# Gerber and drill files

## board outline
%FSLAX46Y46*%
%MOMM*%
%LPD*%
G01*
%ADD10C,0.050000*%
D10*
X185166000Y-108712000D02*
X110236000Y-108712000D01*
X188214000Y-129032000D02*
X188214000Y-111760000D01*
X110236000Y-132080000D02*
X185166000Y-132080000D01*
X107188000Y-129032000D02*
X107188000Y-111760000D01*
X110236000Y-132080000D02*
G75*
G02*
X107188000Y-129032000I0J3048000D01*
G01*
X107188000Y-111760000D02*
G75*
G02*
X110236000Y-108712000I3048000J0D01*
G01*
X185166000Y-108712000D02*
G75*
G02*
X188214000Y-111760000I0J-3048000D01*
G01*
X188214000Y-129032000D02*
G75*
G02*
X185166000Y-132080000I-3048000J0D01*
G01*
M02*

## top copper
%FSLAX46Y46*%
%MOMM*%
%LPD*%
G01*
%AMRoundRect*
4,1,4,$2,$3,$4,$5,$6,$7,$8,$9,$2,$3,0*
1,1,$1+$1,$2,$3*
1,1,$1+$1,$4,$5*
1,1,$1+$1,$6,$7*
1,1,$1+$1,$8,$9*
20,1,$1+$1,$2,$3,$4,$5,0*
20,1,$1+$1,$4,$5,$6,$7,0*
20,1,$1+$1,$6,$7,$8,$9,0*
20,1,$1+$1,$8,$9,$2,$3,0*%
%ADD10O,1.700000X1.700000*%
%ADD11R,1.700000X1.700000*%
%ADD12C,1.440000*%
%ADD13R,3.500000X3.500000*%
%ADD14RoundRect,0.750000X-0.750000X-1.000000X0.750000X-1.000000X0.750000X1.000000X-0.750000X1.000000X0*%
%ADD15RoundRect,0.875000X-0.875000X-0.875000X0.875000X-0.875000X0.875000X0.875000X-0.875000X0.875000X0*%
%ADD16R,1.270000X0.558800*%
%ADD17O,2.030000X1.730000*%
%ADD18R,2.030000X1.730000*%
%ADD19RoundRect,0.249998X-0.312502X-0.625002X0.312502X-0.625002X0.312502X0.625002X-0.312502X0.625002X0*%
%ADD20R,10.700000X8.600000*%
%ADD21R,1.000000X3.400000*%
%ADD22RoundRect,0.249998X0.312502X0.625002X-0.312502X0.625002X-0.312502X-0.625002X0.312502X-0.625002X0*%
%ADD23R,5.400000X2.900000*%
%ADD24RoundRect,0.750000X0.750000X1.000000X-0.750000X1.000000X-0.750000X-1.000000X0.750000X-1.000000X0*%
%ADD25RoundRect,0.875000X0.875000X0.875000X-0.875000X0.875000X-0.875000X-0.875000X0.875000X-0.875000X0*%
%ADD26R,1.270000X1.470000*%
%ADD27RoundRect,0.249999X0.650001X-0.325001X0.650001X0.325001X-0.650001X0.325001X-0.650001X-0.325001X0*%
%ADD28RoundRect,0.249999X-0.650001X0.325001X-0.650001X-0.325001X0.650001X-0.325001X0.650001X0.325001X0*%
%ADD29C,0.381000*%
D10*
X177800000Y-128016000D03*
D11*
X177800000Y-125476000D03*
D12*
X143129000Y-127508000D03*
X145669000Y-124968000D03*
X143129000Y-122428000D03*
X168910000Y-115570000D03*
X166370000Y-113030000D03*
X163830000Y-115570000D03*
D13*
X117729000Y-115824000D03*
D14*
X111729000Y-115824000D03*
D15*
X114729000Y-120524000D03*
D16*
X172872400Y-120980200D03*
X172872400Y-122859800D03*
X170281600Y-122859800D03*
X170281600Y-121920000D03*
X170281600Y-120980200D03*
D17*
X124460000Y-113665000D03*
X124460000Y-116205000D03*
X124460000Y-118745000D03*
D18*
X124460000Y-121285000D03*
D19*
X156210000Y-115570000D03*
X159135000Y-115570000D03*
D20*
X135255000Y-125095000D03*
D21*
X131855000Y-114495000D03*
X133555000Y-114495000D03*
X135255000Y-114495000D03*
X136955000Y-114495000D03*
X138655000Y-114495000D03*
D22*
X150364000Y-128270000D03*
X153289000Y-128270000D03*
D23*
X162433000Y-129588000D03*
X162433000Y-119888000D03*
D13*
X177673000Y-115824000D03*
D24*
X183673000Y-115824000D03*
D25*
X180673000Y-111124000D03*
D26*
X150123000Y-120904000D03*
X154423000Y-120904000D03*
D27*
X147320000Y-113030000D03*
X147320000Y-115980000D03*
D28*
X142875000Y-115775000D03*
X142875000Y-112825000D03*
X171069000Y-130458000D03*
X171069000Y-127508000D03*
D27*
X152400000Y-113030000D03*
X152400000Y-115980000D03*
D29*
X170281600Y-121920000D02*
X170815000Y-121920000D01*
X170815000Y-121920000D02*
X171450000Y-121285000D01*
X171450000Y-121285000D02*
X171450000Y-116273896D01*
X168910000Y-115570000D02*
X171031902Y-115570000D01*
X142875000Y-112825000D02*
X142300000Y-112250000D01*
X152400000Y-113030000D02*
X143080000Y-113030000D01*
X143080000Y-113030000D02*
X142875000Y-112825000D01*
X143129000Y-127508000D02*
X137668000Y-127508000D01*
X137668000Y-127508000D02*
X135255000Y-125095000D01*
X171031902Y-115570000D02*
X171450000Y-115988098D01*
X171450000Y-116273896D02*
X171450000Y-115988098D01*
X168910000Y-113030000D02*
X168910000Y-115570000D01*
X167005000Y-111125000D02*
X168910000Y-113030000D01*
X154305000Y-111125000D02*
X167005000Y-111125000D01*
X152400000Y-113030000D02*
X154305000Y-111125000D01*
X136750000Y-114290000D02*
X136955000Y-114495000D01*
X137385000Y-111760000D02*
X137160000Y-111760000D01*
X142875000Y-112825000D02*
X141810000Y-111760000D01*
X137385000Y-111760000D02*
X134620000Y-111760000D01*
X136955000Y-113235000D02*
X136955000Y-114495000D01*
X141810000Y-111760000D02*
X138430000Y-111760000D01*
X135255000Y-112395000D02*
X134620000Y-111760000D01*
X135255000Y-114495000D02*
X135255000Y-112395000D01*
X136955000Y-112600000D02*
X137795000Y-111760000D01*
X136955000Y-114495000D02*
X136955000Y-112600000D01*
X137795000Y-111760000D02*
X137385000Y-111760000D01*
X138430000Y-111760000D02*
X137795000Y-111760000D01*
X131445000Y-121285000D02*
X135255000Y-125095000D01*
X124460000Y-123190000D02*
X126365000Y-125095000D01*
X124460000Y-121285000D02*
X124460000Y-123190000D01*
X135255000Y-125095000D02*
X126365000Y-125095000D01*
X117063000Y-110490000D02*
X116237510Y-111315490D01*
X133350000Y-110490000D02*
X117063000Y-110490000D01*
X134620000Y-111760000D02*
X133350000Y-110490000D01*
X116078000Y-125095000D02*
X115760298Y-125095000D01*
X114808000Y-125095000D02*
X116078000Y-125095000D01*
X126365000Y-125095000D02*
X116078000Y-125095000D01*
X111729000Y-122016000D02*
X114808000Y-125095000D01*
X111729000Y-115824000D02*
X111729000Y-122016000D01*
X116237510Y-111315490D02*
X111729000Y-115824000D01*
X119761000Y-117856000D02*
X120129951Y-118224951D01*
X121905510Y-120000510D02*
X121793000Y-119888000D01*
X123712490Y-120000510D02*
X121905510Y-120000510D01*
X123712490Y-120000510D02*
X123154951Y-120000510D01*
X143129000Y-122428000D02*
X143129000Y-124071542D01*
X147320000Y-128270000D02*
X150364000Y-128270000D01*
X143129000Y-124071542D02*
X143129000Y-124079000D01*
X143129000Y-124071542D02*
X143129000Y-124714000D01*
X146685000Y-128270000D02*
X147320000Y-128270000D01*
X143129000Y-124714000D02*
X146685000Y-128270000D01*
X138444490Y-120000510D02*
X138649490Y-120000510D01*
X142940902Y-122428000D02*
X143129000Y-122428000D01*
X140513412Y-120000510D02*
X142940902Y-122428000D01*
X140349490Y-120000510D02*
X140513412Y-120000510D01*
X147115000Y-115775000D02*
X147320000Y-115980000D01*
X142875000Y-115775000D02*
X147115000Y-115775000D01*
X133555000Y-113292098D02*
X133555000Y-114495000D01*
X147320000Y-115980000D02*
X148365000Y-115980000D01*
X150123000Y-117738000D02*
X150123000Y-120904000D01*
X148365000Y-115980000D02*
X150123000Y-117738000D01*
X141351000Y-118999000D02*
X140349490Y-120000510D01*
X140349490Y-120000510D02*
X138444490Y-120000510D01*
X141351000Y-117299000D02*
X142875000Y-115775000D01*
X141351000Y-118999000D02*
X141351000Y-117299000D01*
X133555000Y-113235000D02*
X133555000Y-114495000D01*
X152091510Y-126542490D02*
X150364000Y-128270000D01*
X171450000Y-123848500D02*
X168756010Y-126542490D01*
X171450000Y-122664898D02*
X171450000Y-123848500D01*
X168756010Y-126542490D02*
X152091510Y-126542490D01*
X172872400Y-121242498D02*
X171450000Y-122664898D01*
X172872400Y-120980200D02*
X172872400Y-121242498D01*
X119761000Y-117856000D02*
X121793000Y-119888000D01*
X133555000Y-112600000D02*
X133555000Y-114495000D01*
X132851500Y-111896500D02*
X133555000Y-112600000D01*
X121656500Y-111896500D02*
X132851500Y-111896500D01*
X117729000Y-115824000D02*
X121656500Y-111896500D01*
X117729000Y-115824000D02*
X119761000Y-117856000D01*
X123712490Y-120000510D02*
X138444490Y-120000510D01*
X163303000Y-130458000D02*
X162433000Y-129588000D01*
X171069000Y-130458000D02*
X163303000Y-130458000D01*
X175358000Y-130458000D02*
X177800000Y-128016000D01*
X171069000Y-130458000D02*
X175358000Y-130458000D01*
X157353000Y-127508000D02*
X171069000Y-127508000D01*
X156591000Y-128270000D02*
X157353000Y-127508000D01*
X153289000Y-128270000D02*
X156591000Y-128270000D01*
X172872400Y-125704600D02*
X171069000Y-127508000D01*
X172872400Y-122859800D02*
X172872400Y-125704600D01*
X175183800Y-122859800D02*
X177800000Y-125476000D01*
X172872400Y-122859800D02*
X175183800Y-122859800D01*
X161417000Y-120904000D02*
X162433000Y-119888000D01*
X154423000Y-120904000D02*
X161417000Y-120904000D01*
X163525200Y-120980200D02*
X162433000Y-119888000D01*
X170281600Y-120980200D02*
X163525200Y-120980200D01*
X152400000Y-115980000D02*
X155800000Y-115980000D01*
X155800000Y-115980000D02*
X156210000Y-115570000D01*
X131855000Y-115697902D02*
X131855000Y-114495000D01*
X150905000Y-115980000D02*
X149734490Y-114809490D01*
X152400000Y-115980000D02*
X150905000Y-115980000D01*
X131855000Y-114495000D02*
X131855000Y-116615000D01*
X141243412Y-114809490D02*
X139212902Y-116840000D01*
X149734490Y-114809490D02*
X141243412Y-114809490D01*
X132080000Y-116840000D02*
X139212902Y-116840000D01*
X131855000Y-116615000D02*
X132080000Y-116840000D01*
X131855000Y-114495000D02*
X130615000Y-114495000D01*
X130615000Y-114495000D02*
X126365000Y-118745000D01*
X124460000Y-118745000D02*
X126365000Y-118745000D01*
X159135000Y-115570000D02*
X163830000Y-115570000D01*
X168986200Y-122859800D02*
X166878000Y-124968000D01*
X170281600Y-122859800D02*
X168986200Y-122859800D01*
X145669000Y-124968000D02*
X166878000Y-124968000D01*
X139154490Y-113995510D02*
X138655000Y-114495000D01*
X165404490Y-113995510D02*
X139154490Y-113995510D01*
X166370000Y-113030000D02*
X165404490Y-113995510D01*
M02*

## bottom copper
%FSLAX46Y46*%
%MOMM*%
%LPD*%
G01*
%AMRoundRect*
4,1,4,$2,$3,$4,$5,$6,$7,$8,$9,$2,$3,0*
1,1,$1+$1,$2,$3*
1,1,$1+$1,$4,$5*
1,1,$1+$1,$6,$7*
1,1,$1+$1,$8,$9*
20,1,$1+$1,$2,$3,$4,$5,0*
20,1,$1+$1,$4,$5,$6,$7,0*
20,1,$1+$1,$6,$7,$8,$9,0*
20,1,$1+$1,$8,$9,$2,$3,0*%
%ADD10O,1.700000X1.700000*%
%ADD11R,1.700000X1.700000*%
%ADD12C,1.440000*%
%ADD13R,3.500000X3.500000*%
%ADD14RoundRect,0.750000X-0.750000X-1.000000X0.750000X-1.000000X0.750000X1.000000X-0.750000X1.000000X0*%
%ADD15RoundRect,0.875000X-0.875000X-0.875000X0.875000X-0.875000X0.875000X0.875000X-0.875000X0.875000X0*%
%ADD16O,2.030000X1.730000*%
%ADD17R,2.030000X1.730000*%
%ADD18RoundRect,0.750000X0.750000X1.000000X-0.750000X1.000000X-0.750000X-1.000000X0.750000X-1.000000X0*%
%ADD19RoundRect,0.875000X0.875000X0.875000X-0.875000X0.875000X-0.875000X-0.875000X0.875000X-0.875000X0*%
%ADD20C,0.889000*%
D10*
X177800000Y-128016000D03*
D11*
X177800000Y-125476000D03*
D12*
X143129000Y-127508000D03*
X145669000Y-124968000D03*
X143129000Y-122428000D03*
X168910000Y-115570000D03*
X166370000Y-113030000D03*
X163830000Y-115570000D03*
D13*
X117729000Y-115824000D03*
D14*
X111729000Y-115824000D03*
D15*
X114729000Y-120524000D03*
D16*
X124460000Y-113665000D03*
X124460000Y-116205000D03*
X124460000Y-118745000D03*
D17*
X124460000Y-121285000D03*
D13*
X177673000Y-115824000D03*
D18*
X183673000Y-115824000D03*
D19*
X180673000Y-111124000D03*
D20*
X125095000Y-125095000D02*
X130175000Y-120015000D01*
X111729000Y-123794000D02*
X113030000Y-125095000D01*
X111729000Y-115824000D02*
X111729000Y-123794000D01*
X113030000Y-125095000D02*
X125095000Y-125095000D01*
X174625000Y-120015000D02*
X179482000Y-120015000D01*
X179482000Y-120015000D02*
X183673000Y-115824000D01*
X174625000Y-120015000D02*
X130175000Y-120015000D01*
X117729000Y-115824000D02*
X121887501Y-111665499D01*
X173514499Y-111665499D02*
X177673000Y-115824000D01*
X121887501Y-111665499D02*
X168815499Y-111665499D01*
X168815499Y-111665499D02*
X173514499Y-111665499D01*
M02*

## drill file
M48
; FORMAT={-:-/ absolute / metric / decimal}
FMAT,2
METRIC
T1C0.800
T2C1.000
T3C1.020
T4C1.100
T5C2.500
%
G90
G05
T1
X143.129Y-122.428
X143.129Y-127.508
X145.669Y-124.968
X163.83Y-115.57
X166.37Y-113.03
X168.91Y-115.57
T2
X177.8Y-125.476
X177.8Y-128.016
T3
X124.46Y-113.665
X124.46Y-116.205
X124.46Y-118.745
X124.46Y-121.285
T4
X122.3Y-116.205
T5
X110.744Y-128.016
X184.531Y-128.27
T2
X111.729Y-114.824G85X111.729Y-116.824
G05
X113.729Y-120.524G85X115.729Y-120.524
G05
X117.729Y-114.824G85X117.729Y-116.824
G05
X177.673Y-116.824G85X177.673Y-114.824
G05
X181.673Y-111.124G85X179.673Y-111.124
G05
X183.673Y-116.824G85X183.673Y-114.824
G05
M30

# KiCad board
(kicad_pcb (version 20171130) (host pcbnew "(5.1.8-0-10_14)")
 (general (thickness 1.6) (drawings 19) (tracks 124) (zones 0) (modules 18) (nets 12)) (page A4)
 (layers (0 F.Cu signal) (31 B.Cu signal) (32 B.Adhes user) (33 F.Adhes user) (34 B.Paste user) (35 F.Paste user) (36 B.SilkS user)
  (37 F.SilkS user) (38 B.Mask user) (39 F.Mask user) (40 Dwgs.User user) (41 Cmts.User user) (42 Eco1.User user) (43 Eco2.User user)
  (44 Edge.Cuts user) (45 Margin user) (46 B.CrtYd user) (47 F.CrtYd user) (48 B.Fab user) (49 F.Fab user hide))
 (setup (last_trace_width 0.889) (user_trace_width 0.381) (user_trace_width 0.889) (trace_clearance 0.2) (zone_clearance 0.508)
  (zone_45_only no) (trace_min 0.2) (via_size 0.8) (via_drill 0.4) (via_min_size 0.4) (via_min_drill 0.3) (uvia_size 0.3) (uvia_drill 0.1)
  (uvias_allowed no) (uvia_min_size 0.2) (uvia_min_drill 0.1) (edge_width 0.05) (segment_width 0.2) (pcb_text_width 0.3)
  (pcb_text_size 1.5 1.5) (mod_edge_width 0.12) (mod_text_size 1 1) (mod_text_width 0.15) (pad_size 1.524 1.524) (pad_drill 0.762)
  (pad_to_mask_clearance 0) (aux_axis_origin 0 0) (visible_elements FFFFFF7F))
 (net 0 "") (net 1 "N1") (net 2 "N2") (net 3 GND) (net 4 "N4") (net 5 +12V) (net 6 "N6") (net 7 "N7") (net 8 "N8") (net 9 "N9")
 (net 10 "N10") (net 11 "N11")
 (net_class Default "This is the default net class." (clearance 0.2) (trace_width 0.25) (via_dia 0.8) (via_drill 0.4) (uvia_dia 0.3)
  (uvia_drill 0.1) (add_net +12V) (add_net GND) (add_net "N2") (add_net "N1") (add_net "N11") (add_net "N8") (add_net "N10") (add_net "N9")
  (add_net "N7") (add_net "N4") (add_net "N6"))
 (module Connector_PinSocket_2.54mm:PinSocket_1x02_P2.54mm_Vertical (layer F.Cu) (at 177.8 125.476)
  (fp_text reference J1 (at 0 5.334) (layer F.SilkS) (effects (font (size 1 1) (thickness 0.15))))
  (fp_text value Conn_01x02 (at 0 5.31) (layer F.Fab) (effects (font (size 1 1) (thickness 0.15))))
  (pad 2 thru_hole oval (at 0 2.54) (size 1.7 1.7) (drill 1) (layers *.Cu *.Mask) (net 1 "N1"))
  (pad 1 thru_hole rect (at 0 0) (size 1.7 1.7) (drill 1) (layers *.Cu *.Mask) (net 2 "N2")))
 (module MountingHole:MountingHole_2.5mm (layer F.Cu) (at 110.744 128.016)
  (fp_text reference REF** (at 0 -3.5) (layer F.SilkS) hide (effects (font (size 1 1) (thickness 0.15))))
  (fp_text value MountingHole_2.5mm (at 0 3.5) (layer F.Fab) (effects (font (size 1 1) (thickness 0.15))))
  (pad 1 np_thru_hole circle (at 0 0) (size 2.5 2.5) (drill 2.5) (layers *.Cu *.Mask)))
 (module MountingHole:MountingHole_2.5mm (layer F.Cu) (at 184.531 128.27)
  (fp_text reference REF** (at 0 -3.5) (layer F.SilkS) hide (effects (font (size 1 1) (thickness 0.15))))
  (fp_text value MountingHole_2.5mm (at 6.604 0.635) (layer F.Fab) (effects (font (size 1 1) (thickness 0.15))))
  (pad 1 np_thru_hole circle (at 0 0) (size 2.5 2.5) (drill 2.5) (layers *.Cu *.Mask)))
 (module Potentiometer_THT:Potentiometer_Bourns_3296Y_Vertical (layer F.Cu) (at 143.129 122.428 90)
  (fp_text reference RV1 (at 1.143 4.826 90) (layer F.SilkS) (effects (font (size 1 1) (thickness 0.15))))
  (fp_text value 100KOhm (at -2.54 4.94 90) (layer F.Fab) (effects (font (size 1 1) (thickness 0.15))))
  (pad 3 thru_hole circle (at -5.08 0 90) (size 1.44 1.44) (drill 0.8) (layers *.Cu *.Mask) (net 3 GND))
  (pad 2 thru_hole circle (at -2.54 2.54 90) (size 1.44 1.44) (drill 0.8) (layers *.Cu *.Mask) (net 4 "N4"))
  (pad 1 thru_hole circle (at 0 0 90) (size 1.44 1.44) (drill 0.8) (layers *.Cu *.Mask) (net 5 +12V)))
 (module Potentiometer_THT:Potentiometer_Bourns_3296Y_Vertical (layer F.Cu) (at 163.83 115.57 180)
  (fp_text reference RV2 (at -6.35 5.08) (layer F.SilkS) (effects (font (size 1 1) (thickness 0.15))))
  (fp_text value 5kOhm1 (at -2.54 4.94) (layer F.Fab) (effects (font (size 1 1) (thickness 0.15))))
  (pad 3 thru_hole circle (at -5.08 0 180) (size 1.44 1.44) (drill 0.8) (layers *.Cu *.Mask) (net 3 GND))
  (pad 2 thru_hole circle (at -2.54 2.54 180) (size 1.44 1.44) (drill 0.8) (layers *.Cu *.Mask) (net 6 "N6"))
  (pad 1 thru_hole circle (at 0 0 180) (size 1.44 1.44) (drill 0.8) (layers *.Cu *.Mask) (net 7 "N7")))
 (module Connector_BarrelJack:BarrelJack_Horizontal (layer F.Cu) (at 117.729 115.824)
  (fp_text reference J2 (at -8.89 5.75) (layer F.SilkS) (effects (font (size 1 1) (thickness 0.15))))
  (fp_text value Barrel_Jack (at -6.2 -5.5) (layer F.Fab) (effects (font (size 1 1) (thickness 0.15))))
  (pad 1 thru_hole rect (at 0 0) (size 3.5 3.5) (drill oval 1 3) (layers *.Cu *.Mask) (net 5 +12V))
  (pad 2 thru_hole roundrect (at -6 0) (size 3 3.5) (drill oval 1 3) (layers *.Cu *.Mask) (roundrect_rratio 0.25) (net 3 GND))
  (pad 3 thru_hole roundrect (at -3 4.7) (size 3.5 3.5) (drill oval 3 1) (layers *.Cu *.Mask) (roundrect_rratio 0.25)))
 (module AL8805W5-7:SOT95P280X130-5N (layer F.Cu) (at 171.577 121.92)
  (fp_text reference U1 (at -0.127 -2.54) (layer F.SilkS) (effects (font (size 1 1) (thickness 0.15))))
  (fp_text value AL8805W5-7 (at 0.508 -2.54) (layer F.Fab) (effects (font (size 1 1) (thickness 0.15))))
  (pad 5 smd rect (at 1.2954 -0.9398) (size 1.27 0.5588) (layers F.Cu F.Paste F.Mask) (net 5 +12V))
  (pad 4 smd rect (at 1.2954 0.9398) (size 1.27 0.5588) (layers F.Cu F.Paste F.Mask) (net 2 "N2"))
  (pad 3 smd rect (at -1.2954 0.9398) (size 1.27 0.5588) (layers F.Cu F.Paste F.Mask) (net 4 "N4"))
  (pad 2 smd rect (at -1.2954 0) (size 1.27 0.5588) (layers F.Cu F.Paste F.Mask) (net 3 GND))
  (pad 1 smd rect (at -1.2954 -0.9398) (size 1.27 0.5588) (layers F.Cu F.Paste F.Mask) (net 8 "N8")))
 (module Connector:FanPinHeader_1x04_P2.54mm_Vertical (layer F.Cu) (at 124.46 121.285 90)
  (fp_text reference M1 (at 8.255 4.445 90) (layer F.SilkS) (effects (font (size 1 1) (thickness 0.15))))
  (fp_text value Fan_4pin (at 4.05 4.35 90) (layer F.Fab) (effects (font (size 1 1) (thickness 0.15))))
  (pad "" np_thru_hole circle (at 5.08 -2.16 180) (size 1.1 1.1) (drill 1.1) (layers *.Cu *.Mask))
  (pad 4 thru_hole oval (at 7.62 0 180) (size 2.03 1.73) (drill 1.02) (layers *.Cu *.Mask) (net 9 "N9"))
  (pad 3 thru_hole oval (at 5.08 0 180) (size 2.03 1.73) (drill 1.02) (layers *.Cu *.Mask) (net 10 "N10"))
  (pad 2 thru_hole oval (at 2.54 0 180) (size 2.03 1.73) (drill 1.02) (layers *.Cu *.Mask) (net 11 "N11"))
  (pad 1 thru_hole rect (at 0 0 180) (size 2.03 1.73) (drill 1.02) (layers *.Cu *.Mask) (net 3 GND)))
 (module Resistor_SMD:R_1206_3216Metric (layer F.Cu) (at 157.6725 115.57)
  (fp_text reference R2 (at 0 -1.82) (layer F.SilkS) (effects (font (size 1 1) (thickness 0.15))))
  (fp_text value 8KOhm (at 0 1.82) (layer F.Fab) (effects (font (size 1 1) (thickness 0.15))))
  (pad 1 smd roundrect (at -1.4625 0) (size 1.125 1.75) (layers F.Cu F.Paste F.Mask) (roundrect_rratio 0.2222204444444444) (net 11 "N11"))
  (pad 2 smd roundrect (at 1.4625 0) (size 1.125 1.75) (layers F.Cu F.Paste F.Mask) (roundrect_rratio 0.2222204444444444) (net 7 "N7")))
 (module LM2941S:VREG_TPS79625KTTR (layer F.Cu) (at 135.255 125.095 270)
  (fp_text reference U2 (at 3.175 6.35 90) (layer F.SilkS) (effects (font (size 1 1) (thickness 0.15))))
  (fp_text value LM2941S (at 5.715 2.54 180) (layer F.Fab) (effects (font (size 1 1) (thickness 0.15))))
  (pad 6 smd rect (at 0 0 270) (size 8.6 10.7) (layers F.Cu) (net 3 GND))
  (pad 5 smd rect (at -10.6 3.4 270) (size 3.4 1) (layers F.Cu) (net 11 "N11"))
  (pad 4 smd rect (at -10.6 1.7 270) (size 3.4 1) (layers F.Cu) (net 5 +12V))
  (pad 3 smd rect (at -10.6 0 270) (size 3.4 1) (layers F.Cu) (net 3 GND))
  (pad 2 smd rect (at -10.6 -1.7 270) (size 3.4 1) (layers F.Cu) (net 3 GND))
  (pad 1 smd rect (at -10.6 -3.4 270) (size 3.4 1) (layers F.Cu) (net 6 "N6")))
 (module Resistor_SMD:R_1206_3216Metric (layer F.Cu) (at 151.8265 128.27 180)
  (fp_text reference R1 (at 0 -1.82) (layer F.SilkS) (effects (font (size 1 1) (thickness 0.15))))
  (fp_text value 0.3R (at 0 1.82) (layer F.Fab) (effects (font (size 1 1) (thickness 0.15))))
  (pad 2 smd roundrect (at 1.4625 0 180) (size 1.125 1.75) (layers F.Cu F.Paste F.Mask) (roundrect_rratio 0.2222204444444444) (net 5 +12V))
  (pad 1 smd roundrect (at -1.4625 0 180) (size 1.125 1.75) (layers F.Cu F.Paste F.Mask) (roundrect_rratio 0.2222204444444444) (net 2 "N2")))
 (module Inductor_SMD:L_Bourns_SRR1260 (layer F.Cu) (at 162.433 124.738 90)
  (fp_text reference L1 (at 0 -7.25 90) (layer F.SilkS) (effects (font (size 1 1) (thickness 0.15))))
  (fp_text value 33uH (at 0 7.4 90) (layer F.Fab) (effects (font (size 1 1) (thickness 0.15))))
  (pad 1 smd rect (at -4.85 0 90) (size 2.9 5.4) (layers F.Cu F.Paste F.Mask) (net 1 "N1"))
  (pad 2 smd rect (at 4.85 0 90) (size 2.9 5.4) (layers F.Cu F.Paste F.Mask) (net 8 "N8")))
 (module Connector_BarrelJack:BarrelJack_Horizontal (layer F.Cu) (at 177.673 115.824 180)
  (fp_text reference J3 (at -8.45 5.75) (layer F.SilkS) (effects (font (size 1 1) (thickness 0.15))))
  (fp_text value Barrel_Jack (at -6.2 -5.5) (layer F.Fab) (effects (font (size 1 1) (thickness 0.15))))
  (pad 1 thru_hole rect (at 0 0 180) (size 3.5 3.5) (drill oval 1 3) (layers *.Cu *.Mask) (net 5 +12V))
  (pad 2 thru_hole roundrect (at -6 0 180) (size 3 3.5) (drill oval 1 3) (layers *.Cu *.Mask) (roundrect_rratio 0.25) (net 3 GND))
  (pad 3 thru_hole roundrect (at -3 4.7 180) (size 3.5 3.5) (drill oval 3 1) (layers *.Cu *.Mask) (roundrect_rratio 0.25)))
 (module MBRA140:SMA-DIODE (layer F.Cu) (at 152.273 120.904 180)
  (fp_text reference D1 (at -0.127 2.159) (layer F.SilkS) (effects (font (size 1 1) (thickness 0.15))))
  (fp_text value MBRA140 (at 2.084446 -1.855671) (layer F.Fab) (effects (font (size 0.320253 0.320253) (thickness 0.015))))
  (pad C smd rect (at 2.15 0 180) (size 1.27 1.47) (layers F.Cu F.Paste F.Mask) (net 5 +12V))
  (pad A smd rect (at -2.15 0 180) (size 1.27 1.47) (layers F.Cu F.Paste F.Mask) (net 8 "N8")))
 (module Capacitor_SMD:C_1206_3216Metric (layer F.Cu) (at 147.32 114.505 90)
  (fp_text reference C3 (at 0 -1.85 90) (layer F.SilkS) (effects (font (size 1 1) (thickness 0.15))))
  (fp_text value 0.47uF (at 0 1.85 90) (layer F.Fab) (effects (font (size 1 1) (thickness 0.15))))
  (pad 2 smd roundrect (at 1.475 0 90) (size 1.15 1.8) (layers F.Cu F.Paste F.Mask) (roundrect_rratio 0.2173904347826087) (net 3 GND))
  (pad 1 smd roundrect (at -1.475 0 90) (size 1.15 1.8) (layers F.Cu F.Paste F.Mask) (roundrect_rratio 0.2173904347826087) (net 5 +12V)))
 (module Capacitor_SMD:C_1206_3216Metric (layer F.Cu) (at 142.875 114.3 270)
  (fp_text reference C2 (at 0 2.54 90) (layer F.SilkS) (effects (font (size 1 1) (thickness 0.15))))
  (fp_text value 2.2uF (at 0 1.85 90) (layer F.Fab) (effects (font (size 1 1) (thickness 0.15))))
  (pad 2 smd roundrect (at 1.475 0 270) (size 1.15 1.8) (layers F.Cu F.Paste F.Mask) (roundrect_rratio 0.2173904347826087) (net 5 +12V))
  (pad 1 smd roundrect (at -1.475 0 270) (size 1.15 1.8) (layers F.Cu F.Paste F.Mask) (roundrect_rratio 0.2173904347826087) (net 3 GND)))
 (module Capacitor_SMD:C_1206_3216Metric (layer F.Cu) (at 171.069 128.983 270)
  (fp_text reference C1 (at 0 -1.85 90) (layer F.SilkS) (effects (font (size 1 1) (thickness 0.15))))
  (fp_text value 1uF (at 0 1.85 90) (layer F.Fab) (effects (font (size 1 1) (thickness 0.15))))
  (pad 2 smd roundrect (at 1.475 0 270) (size 1.15 1.8) (layers F.Cu F.Paste F.Mask) (roundrect_rratio 0.2173904347826087) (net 1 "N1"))
  (pad 1 smd roundrect (at -1.475 0 270) (size 1.15 1.8) (layers F.Cu F.Paste F.Mask) (roundrect_rratio 0.2173904347826087) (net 2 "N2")))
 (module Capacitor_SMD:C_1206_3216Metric (layer F.Cu) (at 152.4 114.505 90)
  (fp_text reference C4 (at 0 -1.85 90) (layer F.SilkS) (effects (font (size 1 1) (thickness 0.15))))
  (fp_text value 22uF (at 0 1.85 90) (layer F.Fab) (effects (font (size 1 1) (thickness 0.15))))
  (pad 2 smd roundrect (at 1.475 0 90) (size 1.15 1.8) (layers F.Cu F.Paste F.Mask) (roundrect_rratio 0.2173904347826087) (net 3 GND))
  (pad 1 smd roundrect (at -1.475 0 90) (size 1.15 1.8) (layers F.Cu F.Paste F.Mask) (roundrect_rratio 0.2173904347826087) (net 11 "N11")))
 (gr_line (start 185.166 108.712) (end 110.236 108.712) (layer Edge.Cuts) (width 0.05))
 (gr_line (start 188.214 129.032) (end 188.214 111.76) (layer Edge.Cuts) (width 0.05))
 (gr_line (start 110.236 132.08) (end 185.166 132.08) (layer Edge.Cuts) (width 0.05))
 (gr_line (start 107.188 129.032) (end 107.188 111.76) (layer Edge.Cuts) (width 0.05))
 (gr_arc (start 110.236 129.032) (end 107.188 129.032) (angle -90) (layer Edge.Cuts) (width 0.05))
 (gr_arc (start 110.236 111.76) (end 110.236 108.712) (angle -90) (layer Edge.Cuts) (width 0.05))
 (gr_arc (start 185.166 111.76) (end 188.214 111.76) (angle -90) (layer Edge.Cuts) (width 0.05))
 (gr_arc (start 185.166 129.032) (end 185.166 132.08) (angle -90) (layer Edge.Cuts) (width 0.05))
 (segment (start 170.2816 121.92) (end 170.815 121.92) (width 0.381) (layer F.Cu) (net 3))
 (segment (start 170.815 121.92) (end 171.45 121.285) (width 0.381) (layer F.Cu) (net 3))
 (segment (start 171.45 121.285) (end 171.45 116.273896) (width 0.381) (layer F.Cu) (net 3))
 (segment (start 168.91 115.57) (end 171.031902 115.57) (width 0.381) (layer F.Cu) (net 3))
 (segment (start 142.875 112.825) (end 142.3 112.25) (width 0.381) (layer F.Cu) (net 3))
 (segment (start 152.4 113.03) (end 143.08 113.03) (width 0.381) (layer F.Cu) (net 3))
 (segment (start 143.08 113.03) (end 142.875 112.825) (width 0.381) (layer F.Cu) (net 3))
 (segment (start 143.129 127.508) (end 137.668 127.508) (width 0.381) (layer F.Cu) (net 3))
 (segment (start 137.668 127.508) (end 135.255 125.095) (width 0.381) (layer F.Cu) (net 3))
 (segment (start 171.031902 115.57) (end 171.45 115.988098) (width 0.381) (layer F.Cu) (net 3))
 (segment (start 171.45 116.273896) (end 171.45 115.988098) (width 0.381) (layer F.Cu) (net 3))
 (segment (start 168.91 113.03) (end 168.91 115.57) (width 0.381) (layer F.Cu) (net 3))
 (segment (start 167.005 111.125) (end 168.91 113.03) (width 0.381) (layer F.Cu) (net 3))
 (segment (start 154.305 111.125) (end 167.005 111.125) (width 0.381) (layer F.Cu) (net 3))
 (segment (start 152.4 113.03) (end 154.305 111.125) (width 0.381) (layer F.Cu) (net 3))
 (segment (start 136.75 114.29) (end 136.955 114.495) (width 0.381) (layer F.Cu) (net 3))
 (segment (start 137.385 111.76) (end 137.16 111.76) (width 0.381) (layer F.Cu) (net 3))
 (segment (start 142.875 112.825) (end 141.81 111.76) (width 0.381) (layer F.Cu) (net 3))
 (segment (start 137.385 111.76) (end 134.62 111.76) (width 0.381) (layer F.Cu) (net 3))
 (segment (start 136.955 113.235) (end 136.955 114.495) (width 0.381) (layer F.Cu) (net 3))
 (segment (start 141.81 111.76) (end 138.43 111.76) (width 0.381) (layer F.Cu) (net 3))
 (segment (start 135.255 112.395) (end 134.62 111.76) (width 0.381) (layer F.Cu) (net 3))
 (segment (start 135.255 114.495) (end 135.255 112.395) (width 0.381) (layer F.Cu) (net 3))
 (segment (start 136.955 112.6) (end 137.795 111.76) (width 0.381) (layer F.Cu) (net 3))
 (segment (start 136.955 114.495) (end 136.955 112.6) (width 0.381) (layer F.Cu) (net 3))
 (segment (start 137.795 111.76) (end 137.385 111.76) (width 0.381) (layer F.Cu) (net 3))
 (segment (start 138.43 111.76) (end 137.795 111.76) (width 0.381) (layer F.Cu) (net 3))
 (segment (start 131.445 121.285) (end 135.255 125.095) (width 0.381) (layer F.Cu) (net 3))
 (segment (start 124.46 123.19) (end 126.365 125.095) (width 0.381) (layer F.Cu) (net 3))
 (segment (start 124.46 121.285) (end 124.46 123.19) (width 0.381) (layer F.Cu) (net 3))
 (segment (start 135.255 125.095) (end 126.365 125.095) (width 0.381) (layer F.Cu) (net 3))
 (segment (start 125.095 125.095) (end 130.175 120.015) (width 0.889) (layer B.Cu) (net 3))
 (segment (start 117.063 110.49) (end 116.23751 111.31549) (width 0.381) (layer F.Cu) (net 3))
 (segment (start 133.35 110.49) (end 117.063 110.49) (width 0.381) (layer F.Cu) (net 3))
 (segment (start 134.62 111.76) (end 133.35 110.49) (width 0.381) (layer F.Cu) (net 3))
 (segment (start 116.078 125.095) (end 115.760298 125.095) (width 0.381) (layer F.Cu) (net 3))
 (segment (start 114.808 125.095) (end 116.078 125.095) (width 0.381) (layer F.Cu) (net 3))
 (segment (start 126.365 125.095) (end 116.078 125.095) (width 0.381) (layer F.Cu) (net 3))
 (segment (start 111.729 123.794) (end 113.03 125.095) (width 0.889) (layer B.Cu) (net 3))
 (segment (start 111.729 122.016) (end 114.808 125.095) (width 0.381) (layer F.Cu) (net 3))
 (segment (start 111.729 115.824) (end 111.729 122.016) (width 0.381) (layer F.Cu) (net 3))
 (segment (start 116.23751 111.31549) (end 111.729 115.824) (width 0.381) (layer F.Cu) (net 3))
 (segment (start 111.729 115.824) (end 111.729 123.794) (width 0.889) (layer B.Cu) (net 3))
 (segment (start 113.03 125.095) (end 125.095 125.095) (width 0.889) (layer B.Cu) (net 3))
 (segment (start 174.625 120.015) (end 179.482 120.015) (width 0.889) (layer B.Cu) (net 3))
 (segment (start 179.482 120.015) (end 183.673 115.824) (width 0.889) (layer B.Cu) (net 3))
 (segment (start 174.625 120.015) (end 130.175 120.015) (width 0.889) (layer B.Cu) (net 3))
 (segment (start 119.761 117.856) (end 120.129951 118.224951) (width 0.381) (layer F.Cu) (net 5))
 (segment (start 121.90551 120.00051) (end 121.793 119.888) (width 0.381) (layer F.Cu) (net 5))
 (segment (start 123.71249 120.00051) (end 121.90551 120.00051) (width 0.381) (layer F.Cu) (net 5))
 (segment (start 123.71249 120.00051) (end 123.154951 120.00051) (width 0.381) (layer F.Cu) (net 5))
 (segment (start 143.129 122.428) (end 143.129 124.071542) (width 0.381) (layer F.Cu) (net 5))
 (segment (start 147.32 128.27) (end 150.364 128.27) (width 0.381) (layer F.Cu) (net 5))
 (segment (start 143.129 124.071542) (end 143.129 124.079) (width 0.381) (layer F.Cu) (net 5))
 (segment (start 143.129 124.071542) (end 143.129 124.714) (width 0.381) (layer F.Cu) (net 5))
 (segment (start 146.685 128.27) (end 147.32 128.27) (width 0.381) (layer F.Cu) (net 5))
 (segment (start 143.129 124.714) (end 146.685 128.27) (width 0.381) (layer F.Cu) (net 5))
 (segment (start 138.44449 120.00051) (end 138.64949 120.00051) (width 0.381) (layer F.Cu) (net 5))
 (segment (start 142.940902 122.428) (end 143.129 122.428) (width 0.381) (layer F.Cu) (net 5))
 (segment (start 140.513412 120.00051) (end 142.940902 122.428) (width 0.381) (layer F.Cu) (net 5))
 (segment (start 140.34949 120.00051) (end 140.513412 120.00051) (width 0.381) (layer F.Cu) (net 5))
 (segment (start 147.115 115.775) (end 147.32 115.98) (width 0.381) (layer F.Cu) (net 5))
 (segment (start 142.875 115.775) (end 147.115 115.775) (width 0.381) (layer F.Cu) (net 5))
 (segment (start 133.555 113.292098) (end 133.555 114.495) (width 0.381) (layer F.Cu) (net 5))
 (segment (start 147.32 115.98) (end 148.365 115.98) (width 0.381) (layer F.Cu) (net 5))
 (segment (start 150.123 117.738) (end 150.123 120.904) (width 0.381) (layer F.Cu) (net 5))
 (segment (start 148.365 115.98) (end 150.123 117.738) (width 0.381) (layer F.Cu) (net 5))
 (segment (start 141.351 118.999) (end 140.34949 120.00051) (width 0.381) (layer F.Cu) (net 5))
 (segment (start 140.34949 120.00051) (end 138.44449 120.00051) (width 0.381) (layer F.Cu) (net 5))
 (segment (start 141.351 117.299) (end 142.875 115.775) (width 0.381) (layer F.Cu) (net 5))
 (segment (start 141.351 118.999) (end 141.351 117.299) (width 0.381) (layer F.Cu) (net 5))
 (segment (start 133.555 113.235) (end 133.555 114.495) (width 0.381) (layer F.Cu) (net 5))
 (segment (start 152.09151 126.54249) (end 150.364 128.27) (width 0.381) (layer F.Cu) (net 5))
 (segment (start 171.45 123.8485) (end 168.75601 126.54249) (width 0.381) (layer F.Cu) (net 5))
 (segment (start 171.45 122.664898) (end 171.45 123.8485) (width 0.381) (layer F.Cu) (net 5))
 (segment (start 168.75601 126.54249) (end 152.09151 126.54249) (width 0.381) (layer F.Cu) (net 5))
 (segment (start 172.8724 121.242498) (end 171.45 122.664898) (width 0.381) (layer F.Cu) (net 5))
 (segment (start 172.8724 120.9802) (end 172.8724 121.242498) (width 0.381) (layer F.Cu) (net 5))
 (segment (start 119.761 117.856) (end 121.793 119.888) (width 0.381) (layer F.Cu) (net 5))
 (segment (start 133.555 112.6) (end 133.555 114.495) (width 0.381) (layer F.Cu) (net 5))
 (segment (start 132.8515 111.8965) (end 133.555 112.6) (width 0.381) (layer F.Cu) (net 5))
 (segment (start 121.6565 111.8965) (end 132.8515 111.8965) (width 0.381) (layer F.Cu) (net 5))
 (segment (start 117.729 115.824) (end 121.6565 111.8965) (width 0.381) (layer F.Cu) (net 5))
 (segment (start 117.729 115.824) (end 119.761 117.856) (width 0.381) (layer F.Cu) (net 5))
 (segment (start 117.729 115.824) (end 121.887501 111.665499) (width 0.889) (layer B.Cu) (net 5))
 (segment (start 123.71249 120.00051) (end 138.44449 120.00051) (width 0.381) (layer F.Cu) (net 5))
 (segment (start 173.514499 111.665499) (end 177.673 115.824) (width 0.889) (layer B.Cu) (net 5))
 (segment (start 121.887501 111.665499) (end 168.815499 111.665499) (width 0.889) (layer B.Cu) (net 5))
 (segment (start 168.815499 111.665499) (end 173.514499 111.665499) (width 0.889) (layer B.Cu) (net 5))
 (segment (start 163.303 130.458) (end 162.433 129.588) (width 0.381) (layer F.Cu) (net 1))
 (segment (start 171.069 130.458) (end 163.303 130.458) (width 0.381) (layer F.Cu) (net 1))
 (segment (start 175.358 130.458) (end 177.8 128.016) (width 0.381) (layer F.Cu) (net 1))
 (segment (start 171.069 130.458) (end 175.358 130.458) (width 0.381) (layer F.Cu) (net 1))
 (segment (start 157.353 127.508) (end 171.069 127.508) (width 0.381) (layer F.Cu) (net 2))
 (segment (start 156.591 128.27) (end 157.353 127.508) (width 0.381) (layer F.Cu) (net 2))
 (segment (start 153.289 128.27) (end 156.591 128.27) (width 0.381) (layer F.Cu) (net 2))
 (segment (start 172.8724 125.7046) (end 171.069 127.508) (width 0.381) (layer F.Cu) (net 2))
 (segment (start 172.8724 122.8598) (end 172.8724 125.7046) (width 0.381) (layer F.Cu) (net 2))
 (segment (start 175.1838 122.8598) (end 177.8 125.476) (width 0.381) (layer F.Cu) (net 2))
 (segment (start 172.8724 122.8598) (end 175.1838 122.8598) (width 0.381) (layer F.Cu) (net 2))
 (segment (start 161.417 120.904) (end 162.433 119.888) (width 0.381) (layer F.Cu) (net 8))
 (segment (start 154.423 120.904) (end 161.417 120.904) (width 0.381) (layer F.Cu) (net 8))
 (segment (start 163.5252 120.9802) (end 162.433 119.888) (width 0.381) (layer F.Cu) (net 8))
 (segment (start 170.2816 120.9802) (end 163.5252 120.9802) (width 0.381) (layer F.Cu) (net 8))
 (segment (start 152.4 115.98) (end 155.8 115.98) (width 0.381) (layer F.Cu) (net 11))
 (segment (start 155.8 115.98) (end 156.21 115.57) (width 0.381) (layer F.Cu) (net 11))
 (segment (start 131.855 115.697902) (end 131.855 114.495) (width 0.381) (layer F.Cu) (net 11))
 (segment (start 150.905 115.98) (end 149.73449 114.80949) (width 0.381) (layer F.Cu) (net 11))
 (segment (start 152.4 115.98) (end 150.905 115.98) (width 0.381) (layer F.Cu) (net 11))
 (segment (start 131.855 114.495) (end 131.855 116.615) (width 0.381) (layer F.Cu) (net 11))
 (segment (start 141.243412 114.80949) (end 139.212902 116.84) (width 0.381) (layer F.Cu) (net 11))
 (segment (start 149.73449 114.80949) (end 141.243412 114.80949) (width 0.381) (layer F.Cu) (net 11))
 (segment (start 132.08 116.84) (end 139.212902 116.84) (width 0.381) (layer F.Cu) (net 11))
 (segment (start 131.855 116.615) (end 132.08 116.84) (width 0.381) (layer F.Cu) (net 11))
 (segment (start 131.855 114.495) (end 130.615 114.495) (width 0.381) (layer F.Cu) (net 11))
 (segment (start 130.615 114.495) (end 126.365 118.745) (width 0.381) (layer F.Cu) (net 11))
 (segment (start 124.46 118.745) (end 126.365 118.745) (width 0.381) (layer F.Cu) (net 11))
 (segment (start 159.135 115.57) (end 163.83 115.57) (width 0.381) (layer F.Cu) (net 7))
 (segment (start 168.9862 122.8598) (end 166.878 124.968) (width 0.381) (layer F.Cu) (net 4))
 (segment (start 170.2816 122.8598) (end 168.9862 122.8598) (width 0.381) (layer F.Cu) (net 4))
 (segment (start 145.669 124.968) (end 166.878 124.968) (width 0.381) (layer F.Cu) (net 4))
 (segment (start 139.15449 113.99551) (end 138.655 114.495) (width 0.381) (layer F.Cu) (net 6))
 (segment (start 165.40449 113.99551) (end 139.15449 113.99551) (width 0.381) (layer F.Cu) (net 6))
 (segment (start 166.37 113.03) (end 165.40449 113.99551) (width 0.381) (layer F.Cu) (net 6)))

